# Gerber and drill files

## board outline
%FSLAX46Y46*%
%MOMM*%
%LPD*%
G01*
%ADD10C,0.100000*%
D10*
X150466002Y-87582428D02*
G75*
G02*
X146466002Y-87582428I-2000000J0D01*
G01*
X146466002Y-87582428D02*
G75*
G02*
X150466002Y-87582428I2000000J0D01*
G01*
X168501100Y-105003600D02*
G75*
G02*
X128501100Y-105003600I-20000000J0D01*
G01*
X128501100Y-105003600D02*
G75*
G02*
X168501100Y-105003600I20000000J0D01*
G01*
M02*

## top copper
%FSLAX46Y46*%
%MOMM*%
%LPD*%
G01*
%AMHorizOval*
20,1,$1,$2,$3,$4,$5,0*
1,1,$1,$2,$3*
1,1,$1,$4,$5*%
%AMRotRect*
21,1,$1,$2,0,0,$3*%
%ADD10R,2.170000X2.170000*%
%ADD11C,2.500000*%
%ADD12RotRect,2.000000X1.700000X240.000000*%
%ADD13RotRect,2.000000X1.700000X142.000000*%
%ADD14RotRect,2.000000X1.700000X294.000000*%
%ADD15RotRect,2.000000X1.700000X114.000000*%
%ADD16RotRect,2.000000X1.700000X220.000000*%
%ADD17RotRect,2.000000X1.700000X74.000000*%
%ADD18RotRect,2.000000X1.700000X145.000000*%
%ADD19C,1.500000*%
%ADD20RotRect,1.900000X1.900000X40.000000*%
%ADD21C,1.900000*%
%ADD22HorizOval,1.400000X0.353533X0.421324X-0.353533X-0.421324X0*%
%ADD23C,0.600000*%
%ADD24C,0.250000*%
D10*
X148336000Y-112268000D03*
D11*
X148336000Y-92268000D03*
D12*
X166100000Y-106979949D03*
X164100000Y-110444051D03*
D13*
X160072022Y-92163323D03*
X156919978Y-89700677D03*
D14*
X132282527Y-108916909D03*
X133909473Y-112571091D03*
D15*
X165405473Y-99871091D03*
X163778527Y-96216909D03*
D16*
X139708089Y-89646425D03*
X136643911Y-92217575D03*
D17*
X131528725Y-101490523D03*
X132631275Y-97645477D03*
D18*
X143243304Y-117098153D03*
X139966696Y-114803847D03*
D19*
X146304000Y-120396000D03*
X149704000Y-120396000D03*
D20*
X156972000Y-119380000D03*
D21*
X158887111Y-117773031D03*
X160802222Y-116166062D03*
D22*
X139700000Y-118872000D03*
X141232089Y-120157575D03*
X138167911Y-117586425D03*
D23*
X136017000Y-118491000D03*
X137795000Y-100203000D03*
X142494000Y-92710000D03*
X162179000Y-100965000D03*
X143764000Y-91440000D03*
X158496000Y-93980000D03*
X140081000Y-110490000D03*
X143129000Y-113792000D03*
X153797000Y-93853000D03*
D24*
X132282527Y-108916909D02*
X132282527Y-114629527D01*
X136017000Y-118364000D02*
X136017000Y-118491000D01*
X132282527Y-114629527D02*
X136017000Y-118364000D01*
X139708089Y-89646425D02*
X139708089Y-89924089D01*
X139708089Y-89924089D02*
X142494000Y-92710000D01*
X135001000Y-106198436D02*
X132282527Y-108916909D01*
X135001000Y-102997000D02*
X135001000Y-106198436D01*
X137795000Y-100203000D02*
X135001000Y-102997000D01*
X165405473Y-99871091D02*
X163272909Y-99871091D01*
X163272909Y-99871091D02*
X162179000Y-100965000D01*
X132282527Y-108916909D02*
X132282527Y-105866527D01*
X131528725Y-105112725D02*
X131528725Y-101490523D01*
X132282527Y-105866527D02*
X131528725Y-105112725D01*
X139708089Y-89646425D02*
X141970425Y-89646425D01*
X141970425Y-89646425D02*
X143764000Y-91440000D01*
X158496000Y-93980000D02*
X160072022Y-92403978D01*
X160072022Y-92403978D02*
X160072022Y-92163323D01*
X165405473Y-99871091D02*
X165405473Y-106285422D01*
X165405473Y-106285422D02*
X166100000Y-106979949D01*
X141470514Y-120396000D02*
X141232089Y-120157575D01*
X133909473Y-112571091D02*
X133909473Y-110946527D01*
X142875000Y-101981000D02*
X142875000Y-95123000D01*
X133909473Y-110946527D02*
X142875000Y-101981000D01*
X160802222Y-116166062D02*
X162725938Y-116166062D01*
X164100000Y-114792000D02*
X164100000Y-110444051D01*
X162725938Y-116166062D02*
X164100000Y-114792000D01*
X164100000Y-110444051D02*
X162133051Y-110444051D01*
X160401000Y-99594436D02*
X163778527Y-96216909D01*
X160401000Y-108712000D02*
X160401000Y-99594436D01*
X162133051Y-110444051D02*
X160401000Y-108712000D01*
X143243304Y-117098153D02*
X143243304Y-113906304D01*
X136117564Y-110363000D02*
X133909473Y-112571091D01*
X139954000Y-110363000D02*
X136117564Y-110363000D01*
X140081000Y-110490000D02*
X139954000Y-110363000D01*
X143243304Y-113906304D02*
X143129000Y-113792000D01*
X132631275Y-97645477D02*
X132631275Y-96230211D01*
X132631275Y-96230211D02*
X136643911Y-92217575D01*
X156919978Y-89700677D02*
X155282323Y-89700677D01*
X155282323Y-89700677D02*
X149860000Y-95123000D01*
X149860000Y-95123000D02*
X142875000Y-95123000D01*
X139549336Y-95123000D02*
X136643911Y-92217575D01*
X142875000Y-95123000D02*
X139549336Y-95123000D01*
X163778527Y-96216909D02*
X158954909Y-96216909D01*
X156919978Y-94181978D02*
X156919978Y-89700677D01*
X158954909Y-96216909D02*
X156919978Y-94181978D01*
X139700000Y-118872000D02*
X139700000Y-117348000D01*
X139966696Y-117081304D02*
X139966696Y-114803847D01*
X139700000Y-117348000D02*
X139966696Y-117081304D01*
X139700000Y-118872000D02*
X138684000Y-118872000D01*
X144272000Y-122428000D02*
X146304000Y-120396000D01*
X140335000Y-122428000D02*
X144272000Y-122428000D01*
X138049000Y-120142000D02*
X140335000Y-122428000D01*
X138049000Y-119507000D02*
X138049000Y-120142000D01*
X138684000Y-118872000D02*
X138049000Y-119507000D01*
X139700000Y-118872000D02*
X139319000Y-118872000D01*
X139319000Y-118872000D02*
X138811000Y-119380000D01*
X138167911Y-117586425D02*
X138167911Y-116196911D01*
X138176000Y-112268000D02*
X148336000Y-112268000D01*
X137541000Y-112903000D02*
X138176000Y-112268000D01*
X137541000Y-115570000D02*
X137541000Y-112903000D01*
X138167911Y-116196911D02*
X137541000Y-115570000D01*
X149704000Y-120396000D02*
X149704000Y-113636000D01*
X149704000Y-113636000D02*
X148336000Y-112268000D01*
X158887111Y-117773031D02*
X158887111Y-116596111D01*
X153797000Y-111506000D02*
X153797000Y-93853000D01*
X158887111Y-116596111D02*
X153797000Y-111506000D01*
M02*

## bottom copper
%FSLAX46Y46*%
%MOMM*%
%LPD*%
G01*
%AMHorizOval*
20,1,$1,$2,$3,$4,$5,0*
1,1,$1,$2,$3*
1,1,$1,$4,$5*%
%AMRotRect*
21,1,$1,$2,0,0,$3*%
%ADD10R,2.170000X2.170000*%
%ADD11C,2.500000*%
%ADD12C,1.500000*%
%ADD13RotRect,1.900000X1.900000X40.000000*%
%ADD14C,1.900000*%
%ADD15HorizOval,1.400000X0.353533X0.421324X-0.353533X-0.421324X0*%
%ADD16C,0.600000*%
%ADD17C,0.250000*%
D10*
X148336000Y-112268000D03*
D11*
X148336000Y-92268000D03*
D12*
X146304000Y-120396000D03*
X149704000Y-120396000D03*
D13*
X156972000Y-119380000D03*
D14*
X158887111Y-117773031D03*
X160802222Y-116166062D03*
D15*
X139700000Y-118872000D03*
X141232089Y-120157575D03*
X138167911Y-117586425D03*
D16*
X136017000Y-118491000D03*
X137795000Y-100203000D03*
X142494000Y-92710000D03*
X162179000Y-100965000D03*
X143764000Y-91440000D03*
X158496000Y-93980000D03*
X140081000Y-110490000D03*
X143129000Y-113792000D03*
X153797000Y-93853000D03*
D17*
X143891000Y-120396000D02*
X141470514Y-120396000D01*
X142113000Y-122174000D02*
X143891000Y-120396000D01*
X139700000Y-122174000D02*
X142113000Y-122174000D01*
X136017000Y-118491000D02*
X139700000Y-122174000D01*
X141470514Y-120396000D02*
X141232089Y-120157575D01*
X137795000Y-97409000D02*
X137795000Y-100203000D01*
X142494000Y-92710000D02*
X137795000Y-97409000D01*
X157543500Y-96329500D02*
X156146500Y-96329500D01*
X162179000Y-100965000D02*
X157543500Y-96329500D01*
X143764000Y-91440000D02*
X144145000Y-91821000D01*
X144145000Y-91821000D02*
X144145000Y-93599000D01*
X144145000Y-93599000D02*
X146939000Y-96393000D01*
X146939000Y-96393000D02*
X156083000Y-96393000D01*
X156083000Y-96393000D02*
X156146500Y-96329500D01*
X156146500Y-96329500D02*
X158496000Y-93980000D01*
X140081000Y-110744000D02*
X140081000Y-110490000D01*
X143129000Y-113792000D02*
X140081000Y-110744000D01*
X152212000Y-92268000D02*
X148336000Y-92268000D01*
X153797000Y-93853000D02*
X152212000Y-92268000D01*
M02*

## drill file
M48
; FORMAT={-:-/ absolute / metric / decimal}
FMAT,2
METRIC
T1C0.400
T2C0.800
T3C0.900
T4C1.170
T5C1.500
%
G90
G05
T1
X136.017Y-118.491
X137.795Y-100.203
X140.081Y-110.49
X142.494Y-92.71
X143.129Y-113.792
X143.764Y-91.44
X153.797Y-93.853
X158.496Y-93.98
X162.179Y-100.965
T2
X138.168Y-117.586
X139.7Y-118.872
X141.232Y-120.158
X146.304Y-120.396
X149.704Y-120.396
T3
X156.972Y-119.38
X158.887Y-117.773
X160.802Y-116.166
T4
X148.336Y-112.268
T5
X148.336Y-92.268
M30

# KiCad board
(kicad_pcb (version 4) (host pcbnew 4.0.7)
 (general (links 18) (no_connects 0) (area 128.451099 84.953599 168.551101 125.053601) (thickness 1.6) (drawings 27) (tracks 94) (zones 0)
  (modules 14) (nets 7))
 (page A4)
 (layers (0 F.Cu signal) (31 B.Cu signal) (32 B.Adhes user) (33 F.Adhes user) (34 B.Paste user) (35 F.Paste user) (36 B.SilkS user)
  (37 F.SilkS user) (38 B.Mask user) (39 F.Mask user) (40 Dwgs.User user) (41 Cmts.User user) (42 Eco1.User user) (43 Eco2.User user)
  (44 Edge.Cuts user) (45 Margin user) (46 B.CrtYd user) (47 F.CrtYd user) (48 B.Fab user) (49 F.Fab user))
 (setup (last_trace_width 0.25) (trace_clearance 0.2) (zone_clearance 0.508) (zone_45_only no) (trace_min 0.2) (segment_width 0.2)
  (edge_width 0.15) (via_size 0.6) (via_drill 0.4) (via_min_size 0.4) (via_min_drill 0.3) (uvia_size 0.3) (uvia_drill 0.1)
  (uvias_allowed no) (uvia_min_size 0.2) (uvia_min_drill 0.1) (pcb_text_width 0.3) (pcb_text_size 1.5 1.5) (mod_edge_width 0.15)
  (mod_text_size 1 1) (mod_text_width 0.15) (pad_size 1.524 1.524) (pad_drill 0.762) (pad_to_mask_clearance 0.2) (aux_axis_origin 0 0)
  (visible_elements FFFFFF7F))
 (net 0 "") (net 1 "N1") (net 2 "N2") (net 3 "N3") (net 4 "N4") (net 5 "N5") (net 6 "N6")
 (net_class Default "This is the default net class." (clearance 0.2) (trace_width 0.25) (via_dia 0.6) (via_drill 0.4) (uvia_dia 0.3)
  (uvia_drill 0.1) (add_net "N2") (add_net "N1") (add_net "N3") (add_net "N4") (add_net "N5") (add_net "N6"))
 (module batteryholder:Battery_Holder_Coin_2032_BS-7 (layer B.Cu) (at 148.336 112.268 90)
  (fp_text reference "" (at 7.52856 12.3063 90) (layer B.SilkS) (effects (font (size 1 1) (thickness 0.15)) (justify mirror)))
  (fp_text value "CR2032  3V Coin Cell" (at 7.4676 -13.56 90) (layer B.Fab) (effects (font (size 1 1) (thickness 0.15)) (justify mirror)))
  (pad 2 thru_hole rect (at 0 0 90) (size 2.17 2.17) (drill 1.17) (layers *.Cu *.Mask) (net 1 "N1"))
  (pad 1 thru_hole circle (at 20 0 90) (size 2.5 2.5) (drill 1.5) (layers *.Cu *.Mask) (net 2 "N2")))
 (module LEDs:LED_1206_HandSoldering (layer F.Cu) (at 165.1 108.712 240)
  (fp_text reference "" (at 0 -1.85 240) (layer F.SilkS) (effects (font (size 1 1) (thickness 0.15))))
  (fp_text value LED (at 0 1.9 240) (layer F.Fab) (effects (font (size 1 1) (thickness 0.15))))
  (pad 1 smd rect (at -2 0 240) (size 2 1.7) (layers F.Cu F.Paste F.Mask) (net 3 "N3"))
  (pad 2 smd rect (at 2 0 240) (size 2 1.7) (layers F.Cu F.Paste F.Mask) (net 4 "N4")))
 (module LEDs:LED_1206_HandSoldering (layer F.Cu) (at 158.496 90.932 142)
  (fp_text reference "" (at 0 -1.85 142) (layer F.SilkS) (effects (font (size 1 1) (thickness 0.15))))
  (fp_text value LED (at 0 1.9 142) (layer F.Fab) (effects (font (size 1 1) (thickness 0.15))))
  (pad 1 smd rect (at -2 0 142) (size 2 1.7) (layers F.Cu F.Paste F.Mask) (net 3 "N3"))
  (pad 2 smd rect (at 2 0 142) (size 2 1.7) (layers F.Cu F.Paste F.Mask) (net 4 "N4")))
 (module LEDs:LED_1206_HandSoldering (layer F.Cu) (at 133.096 110.744 294)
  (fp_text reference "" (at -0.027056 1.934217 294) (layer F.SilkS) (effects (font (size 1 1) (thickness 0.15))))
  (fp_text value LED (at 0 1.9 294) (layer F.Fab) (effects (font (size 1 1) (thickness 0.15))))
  (pad 1 smd rect (at -2 0 294) (size 2 1.7) (layers F.Cu F.Paste F.Mask) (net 3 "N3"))
  (pad 2 smd rect (at 2 0 294) (size 2 1.7) (layers F.Cu F.Paste F.Mask) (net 4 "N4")))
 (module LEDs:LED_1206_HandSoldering (layer F.Cu) (at 164.592 98.044 114)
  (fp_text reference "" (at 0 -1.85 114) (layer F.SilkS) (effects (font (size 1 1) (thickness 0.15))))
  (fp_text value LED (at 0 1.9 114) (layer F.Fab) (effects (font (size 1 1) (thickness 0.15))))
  (pad 1 smd rect (at -2 0 114) (size 2 1.7) (layers F.Cu F.Paste F.Mask) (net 3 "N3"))
  (pad 2 smd rect (at 2 0 114) (size 2 1.7) (layers F.Cu F.Paste F.Mask) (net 4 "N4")))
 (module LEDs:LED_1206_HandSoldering (layer F.Cu) (at 138.176 90.932 220)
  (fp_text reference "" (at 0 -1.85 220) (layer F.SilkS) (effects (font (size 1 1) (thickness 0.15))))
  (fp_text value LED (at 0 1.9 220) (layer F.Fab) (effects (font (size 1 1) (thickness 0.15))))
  (pad 1 smd rect (at -2 0 220) (size 2 1.7) (layers F.Cu F.Paste F.Mask) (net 3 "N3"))
  (pad 2 smd rect (at 2 0 220) (size 2 1.7) (layers F.Cu F.Paste F.Mask) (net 4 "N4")))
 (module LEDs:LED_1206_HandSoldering (layer F.Cu) (at 132.08 99.568 74)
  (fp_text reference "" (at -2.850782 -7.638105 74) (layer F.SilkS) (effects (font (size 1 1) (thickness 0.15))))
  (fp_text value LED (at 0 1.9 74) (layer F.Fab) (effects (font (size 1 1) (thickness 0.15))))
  (pad 1 smd rect (at -2 0 74) (size 2 1.7) (layers F.Cu F.Paste F.Mask) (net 3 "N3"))
  (pad 2 smd rect (at 2 0 74) (size 2 1.7) (layers F.Cu F.Paste F.Mask) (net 4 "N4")))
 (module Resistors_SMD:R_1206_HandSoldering (layer F.Cu) (at 141.605 115.951 145)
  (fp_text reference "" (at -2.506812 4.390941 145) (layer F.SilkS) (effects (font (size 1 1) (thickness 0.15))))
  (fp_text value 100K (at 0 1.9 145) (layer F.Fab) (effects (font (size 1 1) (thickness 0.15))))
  (pad 1 smd rect (at -2 0 145) (size 2 1.7) (layers F.Cu F.Paste F.Mask) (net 4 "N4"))
  (pad 2 smd rect (at 2 0 145) (size 2 1.7) (layers F.Cu F.Paste F.Mask) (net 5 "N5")))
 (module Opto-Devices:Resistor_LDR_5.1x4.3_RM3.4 (layer F.Cu) (at 146.304 120.396)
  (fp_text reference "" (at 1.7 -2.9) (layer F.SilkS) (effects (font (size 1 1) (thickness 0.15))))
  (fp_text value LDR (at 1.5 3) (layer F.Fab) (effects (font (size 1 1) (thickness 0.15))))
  (pad 1 thru_hole circle (at 0 0) (size 1.5 1.5) (drill 0.8) (layers *.Cu *.Mask) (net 5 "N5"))
  (pad 2 thru_hole circle (at 3.4 0) (size 1.5 1.5) (drill 0.8) (layers *.Cu *.Mask) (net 1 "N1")))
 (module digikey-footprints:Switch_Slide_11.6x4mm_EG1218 (layer F.Cu) (at 156.972 119.38 40)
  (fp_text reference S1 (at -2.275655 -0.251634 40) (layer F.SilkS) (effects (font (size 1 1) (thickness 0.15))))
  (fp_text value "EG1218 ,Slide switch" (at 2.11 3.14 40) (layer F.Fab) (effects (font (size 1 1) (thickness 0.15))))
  (pad 1 thru_hole rect (at 0 0 40) (size 1.9 1.9) (drill 0.9) (layers *.Cu *.Mask) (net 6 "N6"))
  (pad 2 thru_hole circle (at 2.5 0 40) (size 1.9 1.9) (drill 0.9) (layers *.Cu *.Mask) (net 2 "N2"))
  (pad 3 thru_hole circle (at 5 0 40) (size 1.9 1.9) (drill 0.9) (layers *.Cu *.Mask) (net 4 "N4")))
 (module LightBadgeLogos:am (layer F.Cu) (at 158.369 112.522)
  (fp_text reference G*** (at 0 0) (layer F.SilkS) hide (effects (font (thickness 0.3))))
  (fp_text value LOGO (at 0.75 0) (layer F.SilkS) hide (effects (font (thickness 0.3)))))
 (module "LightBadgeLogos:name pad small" (layer F.Cu) (at 149.098 105.029)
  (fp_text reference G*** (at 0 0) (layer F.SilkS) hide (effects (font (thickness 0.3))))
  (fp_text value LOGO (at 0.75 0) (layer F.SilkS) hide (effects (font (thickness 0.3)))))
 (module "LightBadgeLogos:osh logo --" (layer B.Cu) (at 164.211 103.632 180)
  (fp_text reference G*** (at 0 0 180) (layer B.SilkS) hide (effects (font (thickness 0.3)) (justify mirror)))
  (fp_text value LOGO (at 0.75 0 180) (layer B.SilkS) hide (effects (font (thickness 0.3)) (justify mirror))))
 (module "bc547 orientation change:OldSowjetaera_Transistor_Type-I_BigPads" (layer F.Cu) (at 139.7 118.872 140)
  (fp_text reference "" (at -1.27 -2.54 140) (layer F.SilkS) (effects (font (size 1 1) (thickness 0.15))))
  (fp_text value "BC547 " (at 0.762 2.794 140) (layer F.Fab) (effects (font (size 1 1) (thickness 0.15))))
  (pad 1 thru_hole oval (at 0 0 140) (size 1.4 2.5) (drill 0.8) (layers *.Cu *.Mask) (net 5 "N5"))
  (pad 2 thru_hole oval (at -2 0 140) (size 1.4 2.5) (drill 0.8) (layers *.Cu *.Mask) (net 3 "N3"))
  (pad 3 thru_hole oval (at 2 0 140) (size 1.4 2.5) (drill 0.8) (layers *.Cu *.Mask) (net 1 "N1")))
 (gr_circle (center 148.466002 87.582428) (end 150.466002 87.582428) (layer Edge.Cuts) (width 0.1))
 (gr_circle (center 148.5011 105.0036) (end 168.5011 105.0036) (layer Edge.Cuts) (width 0.1))
 (segment (start 132.282527 108.916909) (end 132.282527 114.629527) (width 0.25) (layer F.Cu) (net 3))
 (segment (start 143.891 120.396) (end 141.470514 120.396) (width 0.25) (layer B.Cu) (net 3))
 (segment (start 142.113 122.174) (end 143.891 120.396) (width 0.25) (layer B.Cu) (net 3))
 (segment (start 139.7 122.174) (end 142.113 122.174) (width 0.25) (layer B.Cu) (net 3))
 (segment (start 136.017 118.491) (end 139.7 122.174) (width 0.25) (layer B.Cu) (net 3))
 (via (at 136.017 118.491) (size 0.6) (drill 0.4) (layers F.Cu B.Cu) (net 3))
 (segment (start 136.017 118.364) (end 136.017 118.491) (width 0.25) (layer F.Cu) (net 3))
 (segment (start 132.282527 114.629527) (end 136.017 118.364) (width 0.25) (layer F.Cu) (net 3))
 (segment (start 141.470514 120.396) (end 141.232089 120.157575) (width 0.25) (layer B.Cu) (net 3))
 (segment (start 139.708089 89.646425) (end 139.708089 89.924089) (width 0.25) (layer F.Cu) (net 3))
 (segment (start 139.708089 89.924089) (end 142.494 92.71) (width 0.25) (layer F.Cu) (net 3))
 (segment (start 135.001 106.198436) (end 132.282527 108.916909) (width 0.25) (layer F.Cu) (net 3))
 (segment (start 135.001 102.997) (end 135.001 106.198436) (width 0.25) (layer F.Cu) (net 3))
 (segment (start 137.795 100.203) (end 135.001 102.997) (width 0.25) (layer F.Cu) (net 3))
 (via (at 137.795 100.203) (size 0.6) (drill 0.4) (layers F.Cu B.Cu) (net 3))
 (segment (start 137.795 97.409) (end 137.795 100.203) (width 0.25) (layer B.Cu) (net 3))
 (segment (start 142.494 92.71) (end 137.795 97.409) (width 0.25) (layer B.Cu) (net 3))
 (via (at 142.494 92.71) (size 0.6) (drill 0.4) (layers F.Cu B.Cu) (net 3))
 (segment (start 165.405473 99.871091) (end 163.272909 99.871091) (width 0.25) (layer F.Cu) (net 3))
 (segment (start 157.5435 96.3295) (end 156.1465 96.3295) (width 0.25) (layer B.Cu) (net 3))
 (segment (start 162.179 100.965) (end 157.5435 96.3295) (width 0.25) (layer B.Cu) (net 3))
 (via (at 162.179 100.965) (size 0.6) (drill 0.4) (layers F.Cu B.Cu) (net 3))
 (segment (start 163.272909 99.871091) (end 162.179 100.965) (width 0.25) (layer F.Cu) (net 3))
 (segment (start 132.282527 108.916909) (end 132.282527 105.866527) (width 0.25) (layer F.Cu) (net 3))
 (segment (start 131.528725 105.112725) (end 131.528725 101.490523) (width 0.25) (layer F.Cu) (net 3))
 (segment (start 132.282527 105.866527) (end 131.528725 105.112725) (width 0.25) (layer F.Cu) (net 3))
 (segment (start 139.708089 89.646425) (end 141.970425 89.646425) (width 0.25) (layer F.Cu) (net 3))
 (segment (start 141.970425 89.646425) (end 143.764 91.44) (width 0.25) (layer F.Cu) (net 3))
 (via (at 143.764 91.44) (size 0.6) (drill 0.4) (layers F.Cu B.Cu) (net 3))
 (segment (start 143.764 91.44) (end 144.145 91.821) (width 0.25) (layer B.Cu) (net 3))
 (segment (start 144.145 91.821) (end 144.145 93.599) (width 0.25) (layer B.Cu) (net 3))
 (segment (start 144.145 93.599) (end 146.939 96.393) (width 0.25) (layer B.Cu) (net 3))
 (segment (start 146.939 96.393) (end 156.083 96.393) (width 0.25) (layer B.Cu) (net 3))
 (segment (start 156.083 96.393) (end 156.1465 96.3295) (width 0.25) (layer B.Cu) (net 3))
 (segment (start 158.496 93.98) (end 160.072022 92.403978) (width 0.25) (layer F.Cu) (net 3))
 (segment (start 156.1465 96.3295) (end 158.496 93.98) (width 0.25) (layer B.Cu) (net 3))
 (via (at 158.496 93.98) (size 0.6) (drill 0.4) (layers F.Cu B.Cu) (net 3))
 (segment (start 160.072022 92.403978) (end 160.072022 92.163323) (width 0.25) (layer F.Cu) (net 3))
 (segment (start 165.405473 99.871091) (end 165.405473 106.285422) (width 0.25) (layer F.Cu) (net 3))
 (segment (start 165.405473 106.285422) (end 166.1 106.979949) (width 0.25) (layer F.Cu) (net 3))
 (segment (start 141.470514 120.396) (end 141.232089 120.157575) (width 0.25) (layer F.Cu) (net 3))
 (segment (start 133.909473 112.571091) (end 133.909473 110.946527) (width 0.25) (layer F.Cu) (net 4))
 (segment (start 142.875 101.981) (end 142.875 95.123) (width 0.25) (layer F.Cu) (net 4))
 (segment (start 133.909473 110.946527) (end 142.875 101.981) (width 0.25) (layer F.Cu) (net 4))
 (segment (start 160.802222 116.166062) (end 162.725938 116.166062) (width 0.25) (layer F.Cu) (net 4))
 (segment (start 164.1 114.792) (end 164.1 110.444051) (width 0.25) (layer F.Cu) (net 4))
 (segment (start 162.725938 116.166062) (end 164.1 114.792) (width 0.25) (layer F.Cu) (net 4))
 (segment (start 164.1 110.444051) (end 162.133051 110.444051) (width 0.25) (layer F.Cu) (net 4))
 (segment (start 160.401 99.594436) (end 163.778527 96.216909) (width 0.25) (layer F.Cu) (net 4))
 (segment (start 160.401 108.712) (end 160.401 99.594436) (width 0.25) (layer F.Cu) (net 4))
 (segment (start 162.133051 110.444051) (end 160.401 108.712) (width 0.25) (layer F.Cu) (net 4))
 (segment (start 143.243304 117.098153) (end 143.243304 113.906304) (width 0.25) (layer F.Cu) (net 4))
 (segment (start 136.117564 110.363) (end 133.909473 112.571091) (width 0.25) (layer F.Cu) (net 4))
 (segment (start 139.954 110.363) (end 136.117564 110.363) (width 0.25) (layer F.Cu) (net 4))
 (segment (start 140.081 110.49) (end 139.954 110.363) (width 0.25) (layer F.Cu) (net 4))
 (via (at 140.081 110.49) (size 0.6) (drill 0.4) (layers F.Cu B.Cu) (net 4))
 (segment (start 140.081 110.744) (end 140.081 110.49) (width 0.25) (layer B.Cu) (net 4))
 (segment (start 143.129 113.792) (end 140.081 110.744) (width 0.25) (layer B.Cu) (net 4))
 (via (at 143.129 113.792) (size 0.6) (drill 0.4) (layers F.Cu B.Cu) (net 4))
 (segment (start 143.243304 113.906304) (end 143.129 113.792) (width 0.25) (layer F.Cu) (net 4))
 (segment (start 132.631275 97.645477) (end 132.631275 96.230211) (width 0.25) (layer F.Cu) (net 4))
 (segment (start 132.631275 96.230211) (end 136.643911 92.217575) (width 0.25) (layer F.Cu) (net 4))
 (segment (start 156.919978 89.700677) (end 155.282323 89.700677) (width 0.25) (layer F.Cu) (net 4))
 (segment (start 155.282323 89.700677) (end 149.86 95.123) (width 0.25) (layer F.Cu) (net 4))
 (segment (start 149.86 95.123) (end 142.875 95.123) (width 0.25) (layer F.Cu) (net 4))
 (segment (start 139.549336 95.123) (end 136.643911 92.217575) (width 0.25) (layer F.Cu) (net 4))
 (segment (start 142.875 95.123) (end 139.549336 95.123) (width 0.25) (layer F.Cu) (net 4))
 (segment (start 163.778527 96.216909) (end 158.954909 96.216909) (width 0.25) (layer F.Cu) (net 4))
 (segment (start 156.919978 94.181978) (end 156.919978 89.700677) (width 0.25) (layer F.Cu) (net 4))
 (segment (start 158.954909 96.216909) (end 156.919978 94.181978) (width 0.25) (layer F.Cu) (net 4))
 (segment (start 139.7 118.872) (end 139.7 117.348) (width 0.25) (layer F.Cu) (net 5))
 (segment (start 139.966696 117.081304) (end 139.966696 114.803847) (width 0.25) (layer F.Cu) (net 5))
 (segment (start 139.7 117.348) (end 139.966696 117.081304) (width 0.25) (layer F.Cu) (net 5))
 (segment (start 139.7 118.872) (end 138.684 118.872) (width 0.25) (layer F.Cu) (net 5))
 (segment (start 144.272 122.428) (end 146.304 120.396) (width 0.25) (layer F.Cu) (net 5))
 (segment (start 140.335 122.428) (end 144.272 122.428) (width 0.25) (layer F.Cu) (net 5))
 (segment (start 138.049 120.142) (end 140.335 122.428) (width 0.25) (layer F.Cu) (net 5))
 (segment (start 138.049 119.507) (end 138.049 120.142) (width 0.25) (layer F.Cu) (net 5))
 (segment (start 138.684 118.872) (end 138.049 119.507) (width 0.25) (layer F.Cu) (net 5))
 (segment (start 139.7 118.872) (end 139.319 118.872) (width 0.25) (layer F.Cu) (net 5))
 (segment (start 139.319 118.872) (end 138.811 119.38) (width 0.25) (layer F.Cu) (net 5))
 (segment (start 138.167911 117.586425) (end 138.167911 116.196911) (width 0.25) (layer F.Cu) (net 1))
 (segment (start 138.176 112.268) (end 148.336 112.268) (width 0.25) (layer F.Cu) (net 1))
 (segment (start 137.541 112.903) (end 138.176 112.268) (width 0.25) (layer F.Cu) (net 1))
 (segment (start 137.541 115.57) (end 137.541 112.903) (width 0.25) (layer F.Cu) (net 1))
 (segment (start 138.167911 116.196911) (end 137.541 115.57) (width 0.25) (layer F.Cu) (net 1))
 (segment (start 149.704 120.396) (end 149.704 113.636) (width 0.25) (layer F.Cu) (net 1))
 (segment (start 149.704 113.636) (end 148.336 112.268) (width 0.25) (layer F.Cu) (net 1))
 (segment (start 158.887111 117.773031) (end 158.887111 116.596111) (width 0.25) (layer F.Cu) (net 2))
 (segment (start 152.212 92.268) (end 148.336 92.268) (width 0.25) (layer B.Cu) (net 2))
 (segment (start 153.797 93.853) (end 152.212 92.268) (width 0.25) (layer B.Cu) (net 2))
 (via (at 153.797 93.853) (size 0.6) (drill 0.4) (layers F.Cu B.Cu) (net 2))
 (segment (start 153.797 111.506) (end 153.797 93.853) (width 0.25) (layer F.Cu) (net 2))
 (segment (start 158.887111 116.596111) (end 153.797 111.506) (width 0.25) (layer F.Cu) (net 2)))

